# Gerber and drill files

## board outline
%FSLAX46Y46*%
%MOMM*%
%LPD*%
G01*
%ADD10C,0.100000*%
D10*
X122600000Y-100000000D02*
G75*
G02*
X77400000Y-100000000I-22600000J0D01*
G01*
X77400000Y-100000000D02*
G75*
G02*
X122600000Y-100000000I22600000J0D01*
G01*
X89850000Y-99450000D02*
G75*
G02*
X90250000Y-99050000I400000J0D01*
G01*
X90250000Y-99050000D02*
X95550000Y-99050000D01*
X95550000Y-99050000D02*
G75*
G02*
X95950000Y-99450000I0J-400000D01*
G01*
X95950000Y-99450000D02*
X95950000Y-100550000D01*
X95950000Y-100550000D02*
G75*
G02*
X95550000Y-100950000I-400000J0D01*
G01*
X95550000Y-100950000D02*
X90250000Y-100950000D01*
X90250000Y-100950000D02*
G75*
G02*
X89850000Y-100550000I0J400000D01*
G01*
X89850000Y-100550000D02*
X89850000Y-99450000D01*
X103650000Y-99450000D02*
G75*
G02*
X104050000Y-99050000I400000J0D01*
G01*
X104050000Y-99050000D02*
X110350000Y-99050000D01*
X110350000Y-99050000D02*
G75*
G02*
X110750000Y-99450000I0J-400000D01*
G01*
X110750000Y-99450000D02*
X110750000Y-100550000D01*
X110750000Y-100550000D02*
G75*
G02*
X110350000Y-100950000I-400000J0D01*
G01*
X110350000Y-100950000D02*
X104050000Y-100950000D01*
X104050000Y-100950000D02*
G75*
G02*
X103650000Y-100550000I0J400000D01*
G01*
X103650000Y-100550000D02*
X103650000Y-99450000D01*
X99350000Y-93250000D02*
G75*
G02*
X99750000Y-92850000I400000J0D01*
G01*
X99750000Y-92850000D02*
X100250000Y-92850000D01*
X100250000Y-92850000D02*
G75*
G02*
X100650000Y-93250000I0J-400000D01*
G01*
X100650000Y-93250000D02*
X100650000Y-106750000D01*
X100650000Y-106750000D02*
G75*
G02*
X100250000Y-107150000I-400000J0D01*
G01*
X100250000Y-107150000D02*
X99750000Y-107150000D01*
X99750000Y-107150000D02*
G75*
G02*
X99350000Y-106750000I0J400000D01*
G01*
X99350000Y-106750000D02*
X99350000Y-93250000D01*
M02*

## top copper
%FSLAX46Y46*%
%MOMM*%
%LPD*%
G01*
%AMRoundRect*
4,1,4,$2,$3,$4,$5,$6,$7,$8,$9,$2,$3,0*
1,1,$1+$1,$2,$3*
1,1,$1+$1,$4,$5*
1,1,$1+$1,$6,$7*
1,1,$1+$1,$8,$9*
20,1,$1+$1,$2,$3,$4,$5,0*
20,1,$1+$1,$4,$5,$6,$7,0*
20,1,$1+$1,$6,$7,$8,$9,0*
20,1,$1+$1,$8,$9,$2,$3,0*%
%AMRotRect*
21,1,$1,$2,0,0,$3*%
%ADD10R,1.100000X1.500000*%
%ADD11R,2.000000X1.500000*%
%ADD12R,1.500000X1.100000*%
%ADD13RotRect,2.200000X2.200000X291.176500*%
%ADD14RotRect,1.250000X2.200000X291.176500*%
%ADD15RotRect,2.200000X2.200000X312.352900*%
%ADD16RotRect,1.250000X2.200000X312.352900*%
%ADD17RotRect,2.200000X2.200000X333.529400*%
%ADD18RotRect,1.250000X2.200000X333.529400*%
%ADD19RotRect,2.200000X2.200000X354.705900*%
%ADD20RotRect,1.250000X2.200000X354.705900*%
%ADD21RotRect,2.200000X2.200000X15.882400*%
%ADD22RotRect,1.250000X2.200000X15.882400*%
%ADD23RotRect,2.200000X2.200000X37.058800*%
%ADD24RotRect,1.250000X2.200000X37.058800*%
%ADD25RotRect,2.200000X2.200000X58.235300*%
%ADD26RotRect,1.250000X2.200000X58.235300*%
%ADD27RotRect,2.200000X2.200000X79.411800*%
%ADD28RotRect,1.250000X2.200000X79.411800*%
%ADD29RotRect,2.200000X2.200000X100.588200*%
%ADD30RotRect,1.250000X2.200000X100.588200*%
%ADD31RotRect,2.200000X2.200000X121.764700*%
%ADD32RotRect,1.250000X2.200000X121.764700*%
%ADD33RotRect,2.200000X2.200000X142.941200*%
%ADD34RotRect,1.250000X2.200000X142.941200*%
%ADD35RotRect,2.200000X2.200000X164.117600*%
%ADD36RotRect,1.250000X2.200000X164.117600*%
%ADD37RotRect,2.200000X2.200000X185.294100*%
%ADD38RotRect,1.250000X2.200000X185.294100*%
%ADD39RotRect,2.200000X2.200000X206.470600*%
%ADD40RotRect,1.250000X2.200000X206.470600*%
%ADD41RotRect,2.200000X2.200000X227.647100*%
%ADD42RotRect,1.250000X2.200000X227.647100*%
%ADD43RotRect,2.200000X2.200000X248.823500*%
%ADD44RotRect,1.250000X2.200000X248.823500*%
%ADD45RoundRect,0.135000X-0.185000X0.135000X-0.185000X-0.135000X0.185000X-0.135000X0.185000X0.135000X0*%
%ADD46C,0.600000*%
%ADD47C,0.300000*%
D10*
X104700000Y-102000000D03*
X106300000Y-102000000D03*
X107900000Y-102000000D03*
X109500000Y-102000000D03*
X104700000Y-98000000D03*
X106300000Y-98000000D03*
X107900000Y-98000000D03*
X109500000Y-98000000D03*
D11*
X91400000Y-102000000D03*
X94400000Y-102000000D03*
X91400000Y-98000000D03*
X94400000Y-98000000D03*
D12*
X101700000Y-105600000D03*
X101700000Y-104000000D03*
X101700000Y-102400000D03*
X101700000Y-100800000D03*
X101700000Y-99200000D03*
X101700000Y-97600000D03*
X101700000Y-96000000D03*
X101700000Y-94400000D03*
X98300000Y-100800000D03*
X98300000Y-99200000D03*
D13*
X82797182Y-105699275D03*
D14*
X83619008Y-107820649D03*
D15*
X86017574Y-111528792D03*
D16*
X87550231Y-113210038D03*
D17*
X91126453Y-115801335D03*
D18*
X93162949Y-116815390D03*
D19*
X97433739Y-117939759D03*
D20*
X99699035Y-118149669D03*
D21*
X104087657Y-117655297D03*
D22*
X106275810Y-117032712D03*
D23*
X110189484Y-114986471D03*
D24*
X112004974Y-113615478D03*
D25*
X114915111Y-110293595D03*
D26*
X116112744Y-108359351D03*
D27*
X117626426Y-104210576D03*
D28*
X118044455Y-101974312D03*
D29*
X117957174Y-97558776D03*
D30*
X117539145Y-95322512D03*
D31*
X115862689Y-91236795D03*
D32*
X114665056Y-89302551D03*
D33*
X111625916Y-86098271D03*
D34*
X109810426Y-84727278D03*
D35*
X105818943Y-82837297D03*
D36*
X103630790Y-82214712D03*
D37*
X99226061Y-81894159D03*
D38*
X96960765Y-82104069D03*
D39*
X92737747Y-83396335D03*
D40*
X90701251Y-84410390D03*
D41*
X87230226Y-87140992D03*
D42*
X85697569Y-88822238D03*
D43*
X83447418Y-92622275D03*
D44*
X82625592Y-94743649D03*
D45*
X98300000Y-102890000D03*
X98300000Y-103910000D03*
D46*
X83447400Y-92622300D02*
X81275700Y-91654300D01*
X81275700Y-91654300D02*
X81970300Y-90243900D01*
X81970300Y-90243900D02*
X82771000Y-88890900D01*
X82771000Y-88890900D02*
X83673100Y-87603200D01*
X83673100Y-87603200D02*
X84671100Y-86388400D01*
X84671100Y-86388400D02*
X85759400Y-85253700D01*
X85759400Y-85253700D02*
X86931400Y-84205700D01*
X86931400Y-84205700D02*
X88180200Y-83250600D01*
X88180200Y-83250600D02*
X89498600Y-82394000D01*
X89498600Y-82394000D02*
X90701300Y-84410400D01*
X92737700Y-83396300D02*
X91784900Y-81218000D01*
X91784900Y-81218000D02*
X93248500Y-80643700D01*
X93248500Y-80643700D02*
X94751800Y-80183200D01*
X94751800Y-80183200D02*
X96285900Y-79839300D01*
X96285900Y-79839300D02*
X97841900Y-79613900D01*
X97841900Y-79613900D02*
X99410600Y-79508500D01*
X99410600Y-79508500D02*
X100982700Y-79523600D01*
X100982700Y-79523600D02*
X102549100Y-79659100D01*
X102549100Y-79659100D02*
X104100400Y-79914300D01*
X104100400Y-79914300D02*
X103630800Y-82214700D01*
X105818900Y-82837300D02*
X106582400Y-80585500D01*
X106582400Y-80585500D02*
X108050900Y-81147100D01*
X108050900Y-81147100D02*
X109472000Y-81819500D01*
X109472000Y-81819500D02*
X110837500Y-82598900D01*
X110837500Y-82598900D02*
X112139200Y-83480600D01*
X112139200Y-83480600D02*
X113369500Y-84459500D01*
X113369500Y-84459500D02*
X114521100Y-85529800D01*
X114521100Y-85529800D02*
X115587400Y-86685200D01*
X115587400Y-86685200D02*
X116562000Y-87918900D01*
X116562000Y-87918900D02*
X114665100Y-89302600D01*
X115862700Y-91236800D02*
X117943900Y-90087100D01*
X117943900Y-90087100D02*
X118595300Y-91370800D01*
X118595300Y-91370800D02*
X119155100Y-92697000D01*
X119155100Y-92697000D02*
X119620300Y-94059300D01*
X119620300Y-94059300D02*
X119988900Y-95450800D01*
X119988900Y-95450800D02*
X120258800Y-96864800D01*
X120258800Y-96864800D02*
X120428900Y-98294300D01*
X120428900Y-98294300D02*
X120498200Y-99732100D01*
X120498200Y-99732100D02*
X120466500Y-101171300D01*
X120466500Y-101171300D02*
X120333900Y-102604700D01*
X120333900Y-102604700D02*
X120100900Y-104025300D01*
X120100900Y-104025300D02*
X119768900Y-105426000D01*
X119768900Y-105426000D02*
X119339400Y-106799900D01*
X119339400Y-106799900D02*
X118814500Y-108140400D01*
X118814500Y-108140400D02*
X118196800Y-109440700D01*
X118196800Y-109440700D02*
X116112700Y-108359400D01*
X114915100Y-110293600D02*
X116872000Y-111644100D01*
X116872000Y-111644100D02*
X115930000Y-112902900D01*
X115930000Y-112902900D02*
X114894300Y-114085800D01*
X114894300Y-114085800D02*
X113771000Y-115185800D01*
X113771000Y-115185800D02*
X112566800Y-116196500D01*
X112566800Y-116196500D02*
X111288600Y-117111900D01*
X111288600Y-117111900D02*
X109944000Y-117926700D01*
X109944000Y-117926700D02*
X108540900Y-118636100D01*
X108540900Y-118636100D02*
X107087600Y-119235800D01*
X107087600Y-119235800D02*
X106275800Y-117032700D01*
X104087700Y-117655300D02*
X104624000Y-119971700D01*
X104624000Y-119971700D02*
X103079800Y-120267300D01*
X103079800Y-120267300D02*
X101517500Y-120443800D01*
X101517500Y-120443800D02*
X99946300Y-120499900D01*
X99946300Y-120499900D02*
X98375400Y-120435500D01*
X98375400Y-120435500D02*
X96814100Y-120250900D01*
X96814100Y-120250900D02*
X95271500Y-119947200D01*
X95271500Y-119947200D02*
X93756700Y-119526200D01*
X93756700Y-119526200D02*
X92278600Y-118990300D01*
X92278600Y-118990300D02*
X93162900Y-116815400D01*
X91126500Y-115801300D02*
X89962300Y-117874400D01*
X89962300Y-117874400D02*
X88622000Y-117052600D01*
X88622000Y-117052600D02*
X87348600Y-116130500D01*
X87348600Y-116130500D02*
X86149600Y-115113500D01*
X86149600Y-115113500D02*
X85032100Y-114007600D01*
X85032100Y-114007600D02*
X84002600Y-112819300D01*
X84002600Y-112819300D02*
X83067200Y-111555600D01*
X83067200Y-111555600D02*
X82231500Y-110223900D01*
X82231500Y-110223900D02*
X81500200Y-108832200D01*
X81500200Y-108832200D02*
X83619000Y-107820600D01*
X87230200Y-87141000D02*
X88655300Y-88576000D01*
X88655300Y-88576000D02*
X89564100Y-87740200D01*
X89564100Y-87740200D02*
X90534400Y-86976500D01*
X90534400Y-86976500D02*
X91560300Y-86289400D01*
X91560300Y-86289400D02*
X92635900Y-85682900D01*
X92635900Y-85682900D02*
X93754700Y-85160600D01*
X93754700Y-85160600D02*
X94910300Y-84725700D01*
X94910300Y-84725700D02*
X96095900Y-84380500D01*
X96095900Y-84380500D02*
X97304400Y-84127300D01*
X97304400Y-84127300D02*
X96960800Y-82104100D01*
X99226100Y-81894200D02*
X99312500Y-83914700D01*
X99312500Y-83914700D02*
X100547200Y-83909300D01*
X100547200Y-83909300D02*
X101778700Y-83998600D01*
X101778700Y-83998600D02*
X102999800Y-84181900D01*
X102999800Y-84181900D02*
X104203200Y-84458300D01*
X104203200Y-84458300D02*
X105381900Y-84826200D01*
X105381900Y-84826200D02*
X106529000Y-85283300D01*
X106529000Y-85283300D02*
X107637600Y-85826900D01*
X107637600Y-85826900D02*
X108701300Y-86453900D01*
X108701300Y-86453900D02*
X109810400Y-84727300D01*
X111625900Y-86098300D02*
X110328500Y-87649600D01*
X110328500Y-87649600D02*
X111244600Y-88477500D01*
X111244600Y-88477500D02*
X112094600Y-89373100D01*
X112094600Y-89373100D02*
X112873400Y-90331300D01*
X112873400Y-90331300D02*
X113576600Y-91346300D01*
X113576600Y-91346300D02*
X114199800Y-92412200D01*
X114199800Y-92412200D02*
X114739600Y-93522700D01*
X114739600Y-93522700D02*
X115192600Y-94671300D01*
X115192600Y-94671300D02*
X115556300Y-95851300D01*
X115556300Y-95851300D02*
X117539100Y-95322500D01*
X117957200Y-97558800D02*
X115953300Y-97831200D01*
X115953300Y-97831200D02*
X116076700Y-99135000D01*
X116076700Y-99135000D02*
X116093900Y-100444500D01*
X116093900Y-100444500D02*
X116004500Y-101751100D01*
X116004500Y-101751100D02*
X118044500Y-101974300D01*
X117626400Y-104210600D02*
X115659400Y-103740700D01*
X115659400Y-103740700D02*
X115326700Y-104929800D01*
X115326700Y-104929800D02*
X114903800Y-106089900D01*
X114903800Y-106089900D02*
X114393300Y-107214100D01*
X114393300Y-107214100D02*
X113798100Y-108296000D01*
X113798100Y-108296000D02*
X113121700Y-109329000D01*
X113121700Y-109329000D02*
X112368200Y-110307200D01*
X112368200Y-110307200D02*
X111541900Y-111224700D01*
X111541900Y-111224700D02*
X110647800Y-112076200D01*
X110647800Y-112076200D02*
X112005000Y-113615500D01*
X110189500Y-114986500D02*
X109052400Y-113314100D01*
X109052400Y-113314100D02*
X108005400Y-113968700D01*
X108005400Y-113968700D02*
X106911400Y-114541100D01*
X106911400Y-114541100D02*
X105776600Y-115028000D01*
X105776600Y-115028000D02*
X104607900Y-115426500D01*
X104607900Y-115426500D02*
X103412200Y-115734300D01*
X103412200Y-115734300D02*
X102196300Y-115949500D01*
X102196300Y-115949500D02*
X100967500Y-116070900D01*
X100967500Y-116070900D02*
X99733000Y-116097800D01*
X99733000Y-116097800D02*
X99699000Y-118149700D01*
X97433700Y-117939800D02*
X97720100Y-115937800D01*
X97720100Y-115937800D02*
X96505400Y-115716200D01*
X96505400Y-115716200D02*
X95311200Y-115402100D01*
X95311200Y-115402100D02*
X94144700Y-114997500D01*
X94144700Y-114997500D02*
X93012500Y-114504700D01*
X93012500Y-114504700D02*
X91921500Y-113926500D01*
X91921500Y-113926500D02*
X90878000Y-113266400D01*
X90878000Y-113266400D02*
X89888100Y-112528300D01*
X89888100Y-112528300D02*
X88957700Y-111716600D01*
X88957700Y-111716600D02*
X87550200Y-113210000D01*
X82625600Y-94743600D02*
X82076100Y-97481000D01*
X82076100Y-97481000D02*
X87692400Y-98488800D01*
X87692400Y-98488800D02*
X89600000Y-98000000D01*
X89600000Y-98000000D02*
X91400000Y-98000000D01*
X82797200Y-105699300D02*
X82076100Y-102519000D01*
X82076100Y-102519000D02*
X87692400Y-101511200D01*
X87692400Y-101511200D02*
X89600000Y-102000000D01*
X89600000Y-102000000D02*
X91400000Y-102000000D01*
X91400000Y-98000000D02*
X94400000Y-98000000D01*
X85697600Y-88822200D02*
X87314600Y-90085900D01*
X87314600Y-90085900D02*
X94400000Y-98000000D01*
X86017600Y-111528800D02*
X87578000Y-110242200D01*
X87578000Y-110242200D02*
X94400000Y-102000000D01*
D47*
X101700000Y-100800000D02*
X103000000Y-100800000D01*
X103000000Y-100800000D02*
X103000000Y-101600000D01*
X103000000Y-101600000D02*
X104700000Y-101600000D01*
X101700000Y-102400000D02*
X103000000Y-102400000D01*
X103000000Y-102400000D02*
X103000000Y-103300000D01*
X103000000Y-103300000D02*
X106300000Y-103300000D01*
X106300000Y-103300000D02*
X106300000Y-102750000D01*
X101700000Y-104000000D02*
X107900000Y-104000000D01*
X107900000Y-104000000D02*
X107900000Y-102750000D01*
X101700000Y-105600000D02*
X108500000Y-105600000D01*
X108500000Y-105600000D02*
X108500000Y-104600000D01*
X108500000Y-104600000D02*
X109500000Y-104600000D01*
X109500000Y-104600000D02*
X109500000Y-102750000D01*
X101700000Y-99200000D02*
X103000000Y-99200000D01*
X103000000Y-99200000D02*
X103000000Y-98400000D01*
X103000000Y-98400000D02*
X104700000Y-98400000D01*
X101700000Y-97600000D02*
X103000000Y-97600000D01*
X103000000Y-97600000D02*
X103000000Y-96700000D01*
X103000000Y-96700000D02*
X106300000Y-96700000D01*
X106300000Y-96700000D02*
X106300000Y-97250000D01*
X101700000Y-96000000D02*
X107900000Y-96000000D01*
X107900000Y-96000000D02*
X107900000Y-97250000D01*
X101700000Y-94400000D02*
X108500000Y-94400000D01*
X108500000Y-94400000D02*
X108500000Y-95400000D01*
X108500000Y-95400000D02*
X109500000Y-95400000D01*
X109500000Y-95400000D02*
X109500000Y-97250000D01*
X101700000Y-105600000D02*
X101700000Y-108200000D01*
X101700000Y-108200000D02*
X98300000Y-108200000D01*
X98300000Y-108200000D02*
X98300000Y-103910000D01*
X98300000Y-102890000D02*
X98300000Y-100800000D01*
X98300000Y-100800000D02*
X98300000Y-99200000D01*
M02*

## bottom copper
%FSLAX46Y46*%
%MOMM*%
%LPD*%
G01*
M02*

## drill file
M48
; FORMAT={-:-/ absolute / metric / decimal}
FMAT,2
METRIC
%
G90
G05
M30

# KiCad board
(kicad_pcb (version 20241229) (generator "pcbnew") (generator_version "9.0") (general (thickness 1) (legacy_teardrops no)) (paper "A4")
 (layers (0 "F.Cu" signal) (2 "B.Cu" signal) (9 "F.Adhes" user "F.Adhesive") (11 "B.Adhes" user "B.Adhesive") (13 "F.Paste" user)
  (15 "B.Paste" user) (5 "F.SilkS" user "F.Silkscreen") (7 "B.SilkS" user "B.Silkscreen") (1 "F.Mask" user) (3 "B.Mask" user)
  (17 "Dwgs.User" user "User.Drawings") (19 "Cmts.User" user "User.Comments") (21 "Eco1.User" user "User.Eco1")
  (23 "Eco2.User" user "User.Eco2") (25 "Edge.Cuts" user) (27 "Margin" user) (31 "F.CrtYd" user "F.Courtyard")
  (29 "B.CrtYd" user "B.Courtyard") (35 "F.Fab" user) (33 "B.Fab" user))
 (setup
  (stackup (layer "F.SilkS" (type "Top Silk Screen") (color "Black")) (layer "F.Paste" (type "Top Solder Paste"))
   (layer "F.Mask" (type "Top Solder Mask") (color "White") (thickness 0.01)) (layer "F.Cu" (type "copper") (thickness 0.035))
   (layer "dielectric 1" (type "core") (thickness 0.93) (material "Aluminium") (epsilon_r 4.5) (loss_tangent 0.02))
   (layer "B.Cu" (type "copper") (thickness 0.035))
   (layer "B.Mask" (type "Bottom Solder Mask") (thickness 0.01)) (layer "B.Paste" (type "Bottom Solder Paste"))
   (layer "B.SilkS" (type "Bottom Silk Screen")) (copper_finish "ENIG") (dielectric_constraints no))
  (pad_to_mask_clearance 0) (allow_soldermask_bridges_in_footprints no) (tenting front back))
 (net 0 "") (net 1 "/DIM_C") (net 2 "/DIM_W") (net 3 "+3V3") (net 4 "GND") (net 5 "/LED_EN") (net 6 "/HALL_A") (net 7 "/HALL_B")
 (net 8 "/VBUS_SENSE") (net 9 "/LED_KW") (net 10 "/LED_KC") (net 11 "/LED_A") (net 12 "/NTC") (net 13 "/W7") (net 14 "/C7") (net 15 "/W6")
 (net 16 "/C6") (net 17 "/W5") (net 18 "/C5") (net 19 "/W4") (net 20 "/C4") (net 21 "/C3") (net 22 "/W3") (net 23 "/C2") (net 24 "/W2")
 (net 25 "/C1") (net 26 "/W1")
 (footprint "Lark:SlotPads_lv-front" (layer "F.Cu") (at 100 100)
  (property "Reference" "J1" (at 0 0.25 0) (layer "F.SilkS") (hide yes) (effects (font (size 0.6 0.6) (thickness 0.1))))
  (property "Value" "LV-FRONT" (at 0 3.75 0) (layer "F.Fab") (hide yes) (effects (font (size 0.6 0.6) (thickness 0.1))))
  (pad "1" smd rect (at 4.7 2) (size 1.1 1.5) (layers "F.Cu" "F.Mask") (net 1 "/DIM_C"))
  (pad "2" smd rect (at 6.3 2) (size 1.1 1.5) (layers "F.Cu" "F.Mask") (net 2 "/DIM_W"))
  (pad "3" smd rect (at 7.9 2) (size 1.1 1.5) (layers "F.Cu" "F.Mask") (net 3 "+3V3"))
  (pad "4" smd rect (at 9.5 2) (size 1.1 1.5) (layers "F.Cu" "F.Mask") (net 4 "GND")))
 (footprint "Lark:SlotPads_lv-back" (layer "F.Cu") (at 100 100)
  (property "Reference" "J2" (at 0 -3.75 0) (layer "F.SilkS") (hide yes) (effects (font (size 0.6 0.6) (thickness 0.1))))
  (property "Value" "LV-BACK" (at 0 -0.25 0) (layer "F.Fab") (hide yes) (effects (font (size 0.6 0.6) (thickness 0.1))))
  (pad "1" smd rect (at 4.7 -2) (size 1.1 1.5) (layers "F.Cu" "F.Mask") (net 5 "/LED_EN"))
  (pad "2" smd rect (at 6.3 -2) (size 1.1 1.5) (layers "F.Cu" "F.Mask") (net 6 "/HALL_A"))
  (pad "3" smd rect (at 7.9 -2) (size 1.1 1.5) (layers "F.Cu" "F.Mask") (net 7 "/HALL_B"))
  (pad "4" smd rect (at 9.5 -2) (size 1.1 1.5) (layers "F.Cu" "F.Mask") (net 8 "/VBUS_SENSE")))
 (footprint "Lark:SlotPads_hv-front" (layer "F.Cu") (at 100 100)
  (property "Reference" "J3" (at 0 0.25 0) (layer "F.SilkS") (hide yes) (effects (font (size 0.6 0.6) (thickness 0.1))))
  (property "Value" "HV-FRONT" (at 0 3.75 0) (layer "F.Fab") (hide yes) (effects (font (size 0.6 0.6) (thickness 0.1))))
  (pad "1" smd rect (at -8.6 2) (size 2 1.5) (layers "F.Cu" "F.Mask") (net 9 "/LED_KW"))
  (pad "2" smd rect (at -5.6 2) (size 2 1.5) (layers "F.Cu" "F.Mask") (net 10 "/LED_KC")))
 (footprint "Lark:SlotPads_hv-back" (layer "F.Cu") (at 100 100)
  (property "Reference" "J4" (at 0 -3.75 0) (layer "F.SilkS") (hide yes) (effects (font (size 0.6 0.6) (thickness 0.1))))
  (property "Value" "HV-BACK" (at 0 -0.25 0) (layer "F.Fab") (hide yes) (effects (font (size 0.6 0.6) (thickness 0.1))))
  (pad "1" smd rect (at -8.6 -2) (size 2 1.5) (layers "F.Cu" "F.Mask") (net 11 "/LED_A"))
  (pad "2" smd rect (at -5.6 -2) (size 2 1.5) (layers "F.Cu" "F.Mask") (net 11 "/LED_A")))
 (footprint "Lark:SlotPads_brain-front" (layer "F.Cu") (at 100 100)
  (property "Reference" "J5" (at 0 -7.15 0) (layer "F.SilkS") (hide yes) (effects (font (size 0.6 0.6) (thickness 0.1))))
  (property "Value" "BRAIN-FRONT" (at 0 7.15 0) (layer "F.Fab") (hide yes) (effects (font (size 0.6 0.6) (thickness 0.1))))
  (pad "1" smd rect (at 1.7 5.6) (size 1.5 1.1) (layers "F.Cu" "F.Mask") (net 4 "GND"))
  (pad "2" smd rect (at 1.7 4) (size 1.5 1.1) (layers "F.Cu" "F.Mask") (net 3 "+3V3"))
  (pad "3" smd rect (at 1.7 2.4) (size 1.5 1.1) (layers "F.Cu" "F.Mask") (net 2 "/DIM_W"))
  (pad "4" smd rect (at 1.7 0.8) (size 1.5 1.1) (layers "F.Cu" "F.Mask") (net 1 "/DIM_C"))
  (pad "5" smd rect (at 1.7 -0.8) (size 1.5 1.1) (layers "F.Cu" "F.Mask") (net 5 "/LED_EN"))
  (pad "6" smd rect (at 1.7 -2.4) (size 1.5 1.1) (layers "F.Cu" "F.Mask") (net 6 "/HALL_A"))
  (pad "7" smd rect (at 1.7 -4) (size 1.5 1.1) (layers "F.Cu" "F.Mask") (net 7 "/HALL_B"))
  (pad "8" smd rect (at 1.7 -5.6) (size 1.5 1.1) (layers "F.Cu" "F.Mask") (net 8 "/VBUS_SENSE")))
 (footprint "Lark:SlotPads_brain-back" (layer "F.Cu") (at 100 100)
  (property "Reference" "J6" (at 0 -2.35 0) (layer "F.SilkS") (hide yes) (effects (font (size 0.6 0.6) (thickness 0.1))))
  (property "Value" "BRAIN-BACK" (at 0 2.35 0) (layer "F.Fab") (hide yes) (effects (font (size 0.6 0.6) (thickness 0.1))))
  (pad "1" smd rect (at -1.7 0.8) (size 1.5 1.1) (layers "F.Cu" "F.Mask") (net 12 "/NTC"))
  (pad "2" smd rect (at -1.7 -0.8) (size 1.5 1.1) (layers "F.Cu" "F.Mask") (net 12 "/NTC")))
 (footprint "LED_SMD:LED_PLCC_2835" (layer "F.Cu") (at 83.1223 106.5385 291.1765)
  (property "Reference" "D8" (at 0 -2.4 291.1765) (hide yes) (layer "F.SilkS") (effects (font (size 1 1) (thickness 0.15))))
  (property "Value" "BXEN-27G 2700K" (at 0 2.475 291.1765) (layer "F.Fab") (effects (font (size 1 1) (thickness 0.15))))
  (pad "1" smd rect (at -0.9 0 291.1765) (size 2.2 2.2) (layers "F.Cu" "F.Mask" "F.Paste") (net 9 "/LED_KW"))
  (pad "2" smd rect (at 1.375 0 291.1765) (size 1.25 2.2) (layers "F.Cu" "F.Mask" "F.Paste") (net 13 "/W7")))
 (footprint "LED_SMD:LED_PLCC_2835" (layer "F.Cu") (at 86.6239 112.1939 312.3529)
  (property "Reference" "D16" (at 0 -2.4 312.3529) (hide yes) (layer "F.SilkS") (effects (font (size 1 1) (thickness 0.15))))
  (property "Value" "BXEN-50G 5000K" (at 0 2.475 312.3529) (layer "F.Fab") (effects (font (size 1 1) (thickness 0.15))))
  (pad "1" smd rect (at -0.9 0 312.3529) (size 2.2 2.2) (layers "F.Cu" "F.Mask" "F.Paste") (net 10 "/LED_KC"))
  (pad "2" smd rect (at 1.375 0 312.3529) (size 1.25 2.2) (layers "F.Cu" "F.Mask" "F.Paste") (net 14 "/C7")))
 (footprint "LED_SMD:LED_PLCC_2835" (layer "F.Cu") (at 91.9321 116.2025 333.5294)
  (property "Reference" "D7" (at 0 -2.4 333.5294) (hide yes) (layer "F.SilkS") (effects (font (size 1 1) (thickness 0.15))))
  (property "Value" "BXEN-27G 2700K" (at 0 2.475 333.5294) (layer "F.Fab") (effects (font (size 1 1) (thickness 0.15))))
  (pad "1" smd rect (at -0.9 0 333.5294) (size 2.2 2.2) (layers "F.Cu" "F.Mask" "F.Paste") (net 13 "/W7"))
  (pad "2" smd rect (at 1.375 0 333.5294) (size 1.25 2.2) (layers "F.Cu" "F.Mask" "F.Paste") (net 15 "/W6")))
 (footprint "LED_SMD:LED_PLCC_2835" (layer "F.Cu") (at 98.3299 118.0228 354.7059)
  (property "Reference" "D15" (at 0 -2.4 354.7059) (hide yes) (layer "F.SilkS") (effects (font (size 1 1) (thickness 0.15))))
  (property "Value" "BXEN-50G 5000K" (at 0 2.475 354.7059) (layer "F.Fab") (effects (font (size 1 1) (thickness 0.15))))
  (pad "1" smd rect (at -0.9 0 354.7059) (size 2.2 2.2) (layers "F.Cu" "F.Mask" "F.Paste") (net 14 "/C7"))
  (pad "2" smd rect (at 1.375 0 354.7059) (size 1.25 2.2) (layers "F.Cu" "F.Mask" "F.Paste") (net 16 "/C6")))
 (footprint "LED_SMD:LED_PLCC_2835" (layer "F.Cu") (at 104.9533 117.409 15.8824)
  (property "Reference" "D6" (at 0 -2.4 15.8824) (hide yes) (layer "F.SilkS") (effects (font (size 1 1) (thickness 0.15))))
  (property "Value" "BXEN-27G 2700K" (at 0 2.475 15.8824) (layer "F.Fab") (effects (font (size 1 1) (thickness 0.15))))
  (pad "1" smd rect (at -0.9 0 15.8824) (size 2.2 2.2) (layers "F.Cu" "F.Mask" "F.Paste") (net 15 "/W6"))
  (pad "2" smd rect (at 1.375 0 15.8824) (size 1.25 2.2) (layers "F.Cu" "F.Mask" "F.Paste") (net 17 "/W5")))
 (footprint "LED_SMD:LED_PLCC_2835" (layer "F.Cu") (at 110.9077 114.4441 37.0588)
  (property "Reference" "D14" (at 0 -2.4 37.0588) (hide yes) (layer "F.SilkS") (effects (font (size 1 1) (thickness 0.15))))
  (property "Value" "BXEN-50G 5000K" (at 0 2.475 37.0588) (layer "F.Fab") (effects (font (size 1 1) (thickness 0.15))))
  (pad "1" smd rect (at -0.9 0 37.0588) (size 2.2 2.2) (layers "F.Cu" "F.Mask" "F.Paste") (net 16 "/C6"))
  (pad "2" smd rect (at 1.375 0 37.0588) (size 1.25 2.2) (layers "F.Cu" "F.Mask" "F.Paste") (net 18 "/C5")))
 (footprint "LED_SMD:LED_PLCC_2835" (layer "F.Cu") (at 115.3889 109.5284 58.2353)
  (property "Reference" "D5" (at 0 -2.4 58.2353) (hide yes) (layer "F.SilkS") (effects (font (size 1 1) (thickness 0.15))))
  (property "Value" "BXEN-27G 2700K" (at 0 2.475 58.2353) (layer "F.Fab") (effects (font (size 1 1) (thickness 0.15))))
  (pad "1" smd rect (at -0.9 0 58.2353) (size 2.2 2.2) (layers "F.Cu" "F.Mask" "F.Paste") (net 17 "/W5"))
  (pad "2" smd rect (at 1.375 0 58.2353) (size 1.25 2.2) (layers "F.Cu" "F.Mask" "F.Paste") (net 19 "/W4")))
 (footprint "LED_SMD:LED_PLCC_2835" (layer "F.Cu") (at 117.7918 103.3259 79.4118)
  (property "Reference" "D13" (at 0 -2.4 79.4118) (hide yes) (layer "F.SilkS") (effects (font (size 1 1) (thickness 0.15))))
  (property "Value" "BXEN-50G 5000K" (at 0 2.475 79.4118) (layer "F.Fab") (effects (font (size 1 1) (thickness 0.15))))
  (pad "1" smd rect (at -0.9 0 79.4118) (size 2.2 2.2) (layers "F.Cu" "F.Mask" "F.Paste") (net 18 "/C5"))
  (pad "2" smd rect (at 1.375 0 79.4118) (size 1.25 2.2) (layers "F.Cu" "F.Mask" "F.Paste") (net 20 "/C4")))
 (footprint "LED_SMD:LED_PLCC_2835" (layer "F.Cu") (at 117.7918 96.6741 100.5882)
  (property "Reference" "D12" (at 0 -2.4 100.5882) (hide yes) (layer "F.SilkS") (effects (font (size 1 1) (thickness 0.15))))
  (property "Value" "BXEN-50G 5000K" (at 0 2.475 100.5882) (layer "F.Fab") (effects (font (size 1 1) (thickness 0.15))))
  (pad "1" smd rect (at -0.9 0 100.5882) (size 2.2 2.2) (layers "F.Cu" "F.Mask" "F.Paste") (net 20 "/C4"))
  (pad "2" smd rect (at 1.375 0 100.5882) (size 1.25 2.2) (layers "F.Cu" "F.Mask" "F.Paste") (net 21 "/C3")))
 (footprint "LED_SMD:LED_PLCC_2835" (layer "F.Cu") (at 115.3889 90.4716 121.7647)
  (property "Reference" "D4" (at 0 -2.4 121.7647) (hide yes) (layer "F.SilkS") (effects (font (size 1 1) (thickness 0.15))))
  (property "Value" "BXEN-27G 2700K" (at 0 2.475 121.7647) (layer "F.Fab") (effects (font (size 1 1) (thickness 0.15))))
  (pad "1" smd rect (at -0.9 0 121.7647) (size 2.2 2.2) (layers "F.Cu" "F.Mask" "F.Paste") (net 19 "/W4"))
  (pad "2" smd rect (at 1.375 0 121.7647) (size 1.25 2.2) (layers "F.Cu" "F.Mask" "F.Paste") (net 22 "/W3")))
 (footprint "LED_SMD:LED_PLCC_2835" (layer "F.Cu") (at 110.9077 85.5559 142.9412)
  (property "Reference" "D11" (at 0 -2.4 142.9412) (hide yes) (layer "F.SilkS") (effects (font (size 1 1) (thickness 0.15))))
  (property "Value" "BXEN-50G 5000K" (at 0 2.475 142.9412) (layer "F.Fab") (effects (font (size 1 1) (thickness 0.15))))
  (pad "1" smd rect (at -0.9 0 142.9412) (size 2.2 2.2) (layers "F.Cu" "F.Mask" "F.Paste") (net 21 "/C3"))
  (pad "2" smd rect (at 1.375 0 142.9412) (size 1.25 2.2) (layers "F.Cu" "F.Mask" "F.Paste") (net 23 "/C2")))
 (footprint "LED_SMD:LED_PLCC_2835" (layer "F.Cu") (at 104.9533 82.591 164.1176)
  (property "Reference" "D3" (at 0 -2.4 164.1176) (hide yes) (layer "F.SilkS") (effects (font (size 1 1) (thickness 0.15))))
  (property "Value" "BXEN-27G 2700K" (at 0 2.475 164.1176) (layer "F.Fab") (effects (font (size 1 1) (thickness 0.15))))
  (pad "1" smd rect (at -0.9 0 164.1176) (size 2.2 2.2) (layers "F.Cu" "F.Mask" "F.Paste") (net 22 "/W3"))
  (pad "2" smd rect (at 1.375 0 164.1176) (size 1.25 2.2) (layers "F.Cu" "F.Mask" "F.Paste") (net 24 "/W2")))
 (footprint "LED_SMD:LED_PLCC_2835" (layer "F.Cu") (at 98.3299 81.9772 185.2941)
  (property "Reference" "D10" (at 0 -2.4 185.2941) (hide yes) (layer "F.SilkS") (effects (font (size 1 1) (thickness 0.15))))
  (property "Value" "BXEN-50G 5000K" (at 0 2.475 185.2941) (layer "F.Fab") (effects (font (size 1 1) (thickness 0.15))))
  (pad "1" smd rect (at -0.9 0 185.2941) (size 2.2 2.2) (layers "F.Cu" "F.Mask" "F.Paste") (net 23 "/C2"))
  (pad "2" smd rect (at 1.375 0 185.2941) (size 1.25 2.2) (layers "F.Cu" "F.Mask" "F.Paste") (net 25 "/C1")))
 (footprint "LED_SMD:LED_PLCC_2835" (layer "F.Cu") (at 91.9321 83.7975 206.4706)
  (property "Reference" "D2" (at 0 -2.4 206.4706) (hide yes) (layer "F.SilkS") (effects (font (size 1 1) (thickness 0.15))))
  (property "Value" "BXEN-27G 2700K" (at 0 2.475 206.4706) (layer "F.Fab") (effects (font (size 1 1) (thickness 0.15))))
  (pad "1" smd rect (at -0.9 0 206.4706) (size 2.2 2.2) (layers "F.Cu" "F.Mask" "F.Paste") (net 24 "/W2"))
  (pad "2" smd rect (at 1.375 0 206.4706) (size 1.25 2.2) (layers "F.Cu" "F.Mask" "F.Paste") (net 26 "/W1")))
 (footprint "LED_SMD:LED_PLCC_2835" (layer "F.Cu") (at 86.6239 87.8061 227.6471)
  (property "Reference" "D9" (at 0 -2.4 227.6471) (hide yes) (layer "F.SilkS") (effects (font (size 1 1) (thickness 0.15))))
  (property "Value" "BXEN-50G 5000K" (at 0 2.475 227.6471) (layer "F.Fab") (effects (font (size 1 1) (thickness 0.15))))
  (pad "1" smd rect (at -0.9 0 227.6471) (size 2.2 2.2) (layers "F.Cu" "F.Mask" "F.Paste") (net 25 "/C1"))
  (pad "2" smd rect (at 1.375 0 227.6471) (size 1.25 2.2) (layers "F.Cu" "F.Mask" "F.Paste") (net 11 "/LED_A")))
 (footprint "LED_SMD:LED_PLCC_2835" (layer "F.Cu") (at 83.1223 93.4615 248.8235)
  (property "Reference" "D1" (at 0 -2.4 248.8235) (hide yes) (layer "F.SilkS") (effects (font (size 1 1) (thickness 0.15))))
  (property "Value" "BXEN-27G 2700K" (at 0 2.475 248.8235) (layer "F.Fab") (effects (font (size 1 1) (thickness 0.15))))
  (pad "1" smd rect (at -0.9 0 248.8235) (size 2.2 2.2) (layers "F.Cu" "F.Mask" "F.Paste") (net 26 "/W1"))
  (pad "2" smd rect (at 1.375 0 248.8235) (size 1.25 2.2) (layers "F.Cu" "F.Mask" "F.Paste") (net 11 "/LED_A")))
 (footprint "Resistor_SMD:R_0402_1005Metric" (layer "F.Cu") (at 98.3 103.4 270)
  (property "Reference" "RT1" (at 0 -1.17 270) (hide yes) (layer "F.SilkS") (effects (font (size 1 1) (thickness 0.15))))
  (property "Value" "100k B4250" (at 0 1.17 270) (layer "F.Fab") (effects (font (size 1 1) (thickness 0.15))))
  (pad "1" smd roundrect (at -0.51 0 270) (size 0.54 0.64) (layers "F.Cu" "F.Mask" "F.Paste") (roundrect_rratio 0.25) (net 12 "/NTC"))
  (pad "2" smd roundrect (at 0.51 0 270) (size 0.54 0.64) (layers "F.Cu" "F.Mask" "F.Paste") (roundrect_rratio 0.25) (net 4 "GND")))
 (gr_circle (center 100 100) (end 122.6 100) (stroke (width 0.1) (type default)) (fill no) (layer "Edge.Cuts"))
 (gr_arc (start 89.85 99.45) (mid 89.967157 99.167157) (end 90.25 99.05) (stroke (width 0.1) (type default)) (layer "Edge.Cuts"))
 (gr_line (start 90.25 99.05) (end 95.55 99.05) (stroke (width 0.1) (type default)) (layer "Edge.Cuts"))
 (gr_arc (start 95.55 99.05) (mid 95.832843 99.167157) (end 95.95 99.45) (stroke (width 0.1) (type default)) (layer "Edge.Cuts"))
 (gr_line (start 95.95 99.45) (end 95.95 100.55) (stroke (width 0.1) (type default)) (layer "Edge.Cuts"))
 (gr_arc (start 95.95 100.55) (mid 95.832843 100.832843) (end 95.55 100.95) (stroke (width 0.1) (type default)) (layer "Edge.Cuts"))
 (gr_line (start 95.55 100.95) (end 90.25 100.95) (stroke (width 0.1) (type default)) (layer "Edge.Cuts"))
 (gr_arc (start 90.25 100.95) (mid 89.967157 100.832843) (end 89.85 100.55) (stroke (width 0.1) (type default)) (layer "Edge.Cuts"))
 (gr_line (start 89.85 100.55) (end 89.85 99.45) (stroke (width 0.1) (type default)) (layer "Edge.Cuts"))
 (gr_arc (start 103.65 99.45) (mid 103.767157 99.167157) (end 104.05 99.05) (stroke (width 0.1) (type default)) (layer "Edge.Cuts"))
 (gr_line (start 104.05 99.05) (end 110.35 99.05) (stroke (width 0.1) (type default)) (layer "Edge.Cuts"))
 (gr_arc (start 110.35 99.05) (mid 110.632843 99.167157) (end 110.75 99.45) (stroke (width 0.1) (type default)) (layer "Edge.Cuts"))
 (gr_line (start 110.75 99.45) (end 110.75 100.55) (stroke (width 0.1) (type default)) (layer "Edge.Cuts"))
 (gr_arc (start 110.75 100.55) (mid 110.632843 100.832843) (end 110.35 100.95) (stroke (width 0.1) (type default)) (layer "Edge.Cuts"))
 (gr_line (start 110.35 100.95) (end 104.05 100.95) (stroke (width 0.1) (type default)) (layer "Edge.Cuts"))
 (gr_arc (start 104.05 100.95) (mid 103.767157 100.832843) (end 103.65 100.55) (stroke (width 0.1) (type default)) (layer "Edge.Cuts"))
 (gr_line (start 103.65 100.55) (end 103.65 99.45) (stroke (width 0.1) (type default)) (layer "Edge.Cuts"))
 (gr_arc (start 99.35 93.25) (mid 99.467157 92.967157) (end 99.75 92.85) (stroke (width 0.1) (type default)) (layer "Edge.Cuts"))
 (gr_line (start 99.75 92.85) (end 100.25 92.85) (stroke (width 0.1) (type default)) (layer "Edge.Cuts"))
 (gr_arc (start 100.25 92.85) (mid 100.532843 92.967157) (end 100.65 93.25) (stroke (width 0.1) (type default)) (layer "Edge.Cuts"))
 (gr_line (start 100.65 93.25) (end 100.65 106.75) (stroke (width 0.1) (type default)) (layer "Edge.Cuts"))
 (gr_arc (start 100.65 106.75) (mid 100.532843 107.032843) (end 100.25 107.15) (stroke (width 0.1) (type default)) (layer "Edge.Cuts"))
 (gr_line (start 100.25 107.15) (end 99.75 107.15) (stroke (width 0.1) (type default)) (layer "Edge.Cuts"))
 (gr_arc (start 99.75 107.15) (mid 99.467157 107.032843) (end 99.35 106.75) (stroke (width 0.1) (type default)) (layer "Edge.Cuts"))
 (gr_line (start 99.35 106.75) (end 99.35 93.25) (stroke (width 0.1) (type default)) (layer "Edge.Cuts"))
 (segment (start 83.4474 92.6223) (end 81.2757 91.6543) (width 0.6) (layer "F.Cu") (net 26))
 (segment (start 81.2757 91.6543) (end 81.9703 90.2439) (width 0.6) (layer "F.Cu") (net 26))
 (segment (start 81.9703 90.2439) (end 82.771 88.8909) (width 0.6) (layer "F.Cu") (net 26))
 (segment (start 82.771 88.8909) (end 83.6731 87.6032) (width 0.6) (layer "F.Cu") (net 26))
 (segment (start 83.6731 87.6032) (end 84.6711 86.3884) (width 0.6) (layer "F.Cu") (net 26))
 (segment (start 84.6711 86.3884) (end 85.7594 85.2537) (width 0.6) (layer "F.Cu") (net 26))
 (segment (start 85.7594 85.2537) (end 86.9314 84.2057) (width 0.6) (layer "F.Cu") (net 26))
 (segment (start 86.9314 84.2057) (end 88.1802 83.2506) (width 0.6) (layer "F.Cu") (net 26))
 (segment (start 88.1802 83.2506) (end 89.4986 82.394) (width 0.6) (layer "F.Cu") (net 26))
 (segment (start 89.4986 82.394) (end 90.7013 84.4104) (width 0.6) (layer "F.Cu") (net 26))
 (segment (start 92.7377 83.3963) (end 91.7849 81.218) (width 0.6) (layer "F.Cu") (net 24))
 (segment (start 91.7849 81.218) (end 93.2485 80.6437) (width 0.6) (layer "F.Cu") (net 24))
 (segment (start 93.2485 80.6437) (end 94.7518 80.1832) (width 0.6) (layer "F.Cu") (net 24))
 (segment (start 94.7518 80.1832) (end 96.2859 79.8393) (width 0.6) (layer "F.Cu") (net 24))
 (segment (start 96.2859 79.8393) (end 97.8419 79.6139) (width 0.6) (layer "F.Cu") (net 24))
 (segment (start 97.8419 79.6139) (end 99.4106 79.5085) (width 0.6) (layer "F.Cu") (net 24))
 (segment (start 99.4106 79.5085) (end 100.9827 79.5236) (width 0.6) (layer "F.Cu") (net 24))
 (segment (start 100.9827 79.5236) (end 102.5491 79.6591) (width 0.6) (layer "F.Cu") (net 24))
 (segment (start 102.5491 79.6591) (end 104.1004 79.9143) (width 0.6) (layer "F.Cu") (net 24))
 (segment (start 104.1004 79.9143) (end 103.6308 82.2147) (width 0.6) (layer "F.Cu") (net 24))
 (segment (start 105.8189 82.8373) (end 106.5824 80.5855) (width 0.6) (layer "F.Cu") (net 22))
 (segment (start 106.5824 80.5855) (end 108.0509 81.1471) (width 0.6) (layer "F.Cu") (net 22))
 (segment (start 108.0509 81.1471) (end 109.472 81.8195) (width 0.6) (layer "F.Cu") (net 22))
 (segment (start 109.472 81.8195) (end 110.8375 82.5989) (width 0.6) (layer "F.Cu") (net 22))
 (segment (start 110.8375 82.5989) (end 112.1392 83.4806) (width 0.6) (layer "F.Cu") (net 22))
 (segment (start 112.1392 83.4806) (end 113.3695 84.4595) (width 0.6) (layer "F.Cu") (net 22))
 (segment (start 113.3695 84.4595) (end 114.5211 85.5298) (width 0.6) (layer "F.Cu") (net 22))
 (segment (start 114.5211 85.5298) (end 115.5874 86.6852) (width 0.6) (layer "F.Cu") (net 22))
 (segment (start 115.5874 86.6852) (end 116.562 87.9189) (width 0.6) (layer "F.Cu") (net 22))
 (segment (start 116.562 87.9189) (end 114.6651 89.3026) (width 0.6) (layer "F.Cu") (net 22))
 (segment (start 115.8627 91.2368) (end 117.9439 90.0871) (width 0.6) (layer "F.Cu") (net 19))
 (segment (start 117.9439 90.0871) (end 118.5953 91.3708) (width 0.6) (layer "F.Cu") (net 19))
 (segment (start 118.5953 91.3708) (end 119.1551 92.697) (width 0.6) (layer "F.Cu") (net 19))
 (segment (start 119.1551 92.697) (end 119.6203 94.0593) (width 0.6) (layer "F.Cu") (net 19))
 (segment (start 119.6203 94.0593) (end 119.9889 95.4508) (width 0.6) (layer "F.Cu") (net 19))
 (segment (start 119.9889 95.4508) (end 120.2588 96.8648) (width 0.6) (layer "F.Cu") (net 19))
 (segment (start 120.2588 96.8648) (end 120.4289 98.2943) (width 0.6) (layer "F.Cu") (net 19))
 (segment (start 120.4289 98.2943) (end 120.4982 99.7321) (width 0.6) (layer "F.Cu") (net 19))
 (segment (start 120.4982 99.7321) (end 120.4665 101.1713) (width 0.6) (layer "F.Cu") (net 19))
 (segment (start 120.4665 101.1713) (end 120.3339 102.6047) (width 0.6) (layer "F.Cu") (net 19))
 (segment (start 120.3339 102.6047) (end 120.1009 104.0253) (width 0.6) (layer "F.Cu") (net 19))
 (segment (start 120.1009 104.0253) (end 119.7689 105.426) (width 0.6) (layer "F.Cu") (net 19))
 (segment (start 119.7689 105.426) (end 119.3394 106.7999) (width 0.6) (layer "F.Cu") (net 19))
 (segment (start 119.3394 106.7999) (end 118.8145 108.1404) (width 0.6) (layer "F.Cu") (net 19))
 (segment (start 118.8145 108.1404) (end 118.1968 109.4407) (width 0.6) (layer "F.Cu") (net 19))
 (segment (start 118.1968 109.4407) (end 116.1127 108.3594) (width 0.6) (layer "F.Cu") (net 19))
 (segment (start 114.9151 110.2936) (end 116.872 111.6441) (width 0.6) (layer "F.Cu") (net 17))
 (segment (start 116.872 111.6441) (end 115.93 112.9029) (width 0.6) (layer "F.Cu") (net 17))
 (segment (start 115.93 112.9029) (end 114.8943 114.0858) (width 0.6) (layer "F.Cu") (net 17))
 (segment (start 114.8943 114.0858) (end 113.771 115.1858) (width 0.6) (layer "F.Cu") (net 17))
 (segment (start 113.771 115.1858) (end 112.5668 116.1965) (width 0.6) (layer "F.Cu") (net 17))
 (segment (start 112.5668 116.1965) (end 111.2886 117.1119) (width 0.6) (layer "F.Cu") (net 17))
 (segment (start 111.2886 117.1119) (end 109.944 117.9267) (width 0.6) (layer "F.Cu") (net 17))
 (segment (start 109.944 117.9267) (end 108.5409 118.6361) (width 0.6) (layer "F.Cu") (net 17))
 (segment (start 108.5409 118.6361) (end 107.0876 119.2358) (width 0.6) (layer "F.Cu") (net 17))
 (segment (start 107.0876 119.2358) (end 106.2758 117.0327) (width 0.6) (layer "F.Cu") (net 17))
 (segment (start 104.0877 117.6553) (end 104.624 119.9717) (width 0.6) (layer "F.Cu") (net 15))
 (segment (start 104.624 119.9717) (end 103.0798 120.2673) (width 0.6) (layer "F.Cu") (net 15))
 (segment (start 103.0798 120.2673) (end 101.5175 120.4438) (width 0.6) (layer "F.Cu") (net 15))
 (segment (start 101.5175 120.4438) (end 99.9463 120.4999) (width 0.6) (layer "F.Cu") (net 15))
 (segment (start 99.9463 120.4999) (end 98.3754 120.4355) (width 0.6) (layer "F.Cu") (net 15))
 (segment (start 98.3754 120.4355) (end 96.8141 120.2509) (width 0.6) (layer "F.Cu") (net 15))
 (segment (start 96.8141 120.2509) (end 95.2715 119.9472) (width 0.6) (layer "F.Cu") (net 15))
 (segment (start 95.2715 119.9472) (end 93.7567 119.5262) (width 0.6) (layer "F.Cu") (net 15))
 (segment (start 93.7567 119.5262) (end 92.2786 118.9903) (width 0.6) (layer "F.Cu") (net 15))
 (segment (start 92.2786 118.9903) (end 93.1629 116.8154) (width 0.6) (layer "F.Cu") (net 15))
 (segment (start 91.1265 115.8013) (end 89.9623 117.8744) (width 0.6) (layer "F.Cu") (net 13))
 (segment (start 89.9623 117.8744) (end 88.622 117.0526) (width 0.6) (layer "F.Cu") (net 13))
 (segment (start 88.622 117.0526) (end 87.3486 116.1305) (width 0.6) (layer "F.Cu") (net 13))
 (segment (start 87.3486 116.1305) (end 86.1496 115.1135) (width 0.6) (layer "F.Cu") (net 13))
 (segment (start 86.1496 115.1135) (end 85.0321 114.0076) (width 0.6) (layer "F.Cu") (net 13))
 (segment (start 85.0321 114.0076) (end 84.0026 112.8193) (width 0.6) (layer "F.Cu") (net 13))
 (segment (start 84.0026 112.8193) (end 83.0672 111.5556) (width 0.6) (layer "F.Cu") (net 13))
 (segment (start 83.0672 111.5556) (end 82.2315 110.2239) (width 0.6) (layer "F.Cu") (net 13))
 (segment (start 82.2315 110.2239) (end 81.5002 108.8322) (width 0.6) (layer "F.Cu") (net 13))
 (segment (start 81.5002 108.8322) (end 83.619 107.8206) (width 0.6) (layer "F.Cu") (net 13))
 (segment (start 87.2302 87.141) (end 88.6553 88.576) (width 0.6) (layer "F.Cu") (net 25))
 (segment (start 88.6553 88.576) (end 89.5641 87.7402) (width 0.6) (layer "F.Cu") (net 25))
 (segment (start 89.5641 87.7402) (end 90.5344 86.9765) (width 0.6) (layer "F.Cu") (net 25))
 (segment (start 90.5344 86.9765) (end 91.5603 86.2894) (width 0.6) (layer "F.Cu") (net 25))
 (segment (start 91.5603 86.2894) (end 92.6359 85.6829) (width 0.6) (layer "F.Cu") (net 25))
 (segment (start 92.6359 85.6829) (end 93.7547 85.1606) (width 0.6) (layer "F.Cu") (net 25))
 (segment (start 93.7547 85.1606) (end 94.9103 84.7257) (width 0.6) (layer "F.Cu") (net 25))
 (segment (start 94.9103 84.7257) (end 96.0959 84.3805) (width 0.6) (layer "F.Cu") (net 25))
 (segment (start 96.0959 84.3805) (end 97.3044 84.1273) (width 0.6) (layer "F.Cu") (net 25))
 (segment (start 97.3044 84.1273) (end 96.9608 82.1041) (width 0.6) (layer "F.Cu") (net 25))
 (segment (start 99.2261 81.8942) (end 99.3125 83.9147) (width 0.6) (layer "F.Cu") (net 23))
 (segment (start 99.3125 83.9147) (end 100.5472 83.9093) (width 0.6) (layer "F.Cu") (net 23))
 (segment (start 100.5472 83.9093) (end 101.7787 83.9986) (width 0.6) (layer "F.Cu") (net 23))
 (segment (start 101.7787 83.9986) (end 102.9998 84.1819) (width 0.6) (layer "F.Cu") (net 23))
 (segment (start 102.9998 84.1819) (end 104.2032 84.4583) (width 0.6) (layer "F.Cu") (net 23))
 (segment (start 104.2032 84.4583) (end 105.3819 84.8262) (width 0.6) (layer "F.Cu") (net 23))
 (segment (start 105.3819 84.8262) (end 106.529 85.2833) (width 0.6) (layer "F.Cu") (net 23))
 (segment (start 106.529 85.2833) (end 107.6376 85.8269) (width 0.6) (layer "F.Cu") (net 23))
 (segment (start 107.6376 85.8269) (end 108.7013 86.4539) (width 0.6) (layer "F.Cu") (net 23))
 (segment (start 108.7013 86.4539) (end 109.8104 84.7273) (width 0.6) (layer "F.Cu") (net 23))
 (segment (start 111.6259 86.0983) (end 110.3285 87.6496) (width 0.6) (layer "F.Cu") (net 21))
 (segment (start 110.3285 87.6496) (end 111.2446 88.4775) (width 0.6) (layer "F.Cu") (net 21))
 (segment (start 111.2446 88.4775) (end 112.0946 89.3731) (width 0.6) (layer "F.Cu") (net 21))
 (segment (start 112.0946 89.3731) (end 112.8734 90.3313) (width 0.6) (layer "F.Cu") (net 21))
 (segment (start 112.8734 90.3313) (end 113.5766 91.3463) (width 0.6) (layer "F.Cu") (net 21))
 (segment (start 113.5766 91.3463) (end 114.1998 92.4122) (width 0.6) (layer "F.Cu") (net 21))
 (segment (start 114.1998 92.4122) (end 114.7396 93.5227) (width 0.6) (layer "F.Cu") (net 21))
 (segment (start 114.7396 93.5227) (end 115.1926 94.6713) (width 0.6) (layer "F.Cu") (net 21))
 (segment (start 115.1926 94.6713) (end 115.5563 95.8513) (width 0.6) (layer "F.Cu") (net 21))
 (segment (start 115.5563 95.8513) (end 117.5391 95.3225) (width 0.6) (layer "F.Cu") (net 21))
 (segment (start 117.9572 97.5588) (end 115.9533 97.8312) (width 0.6) (layer "F.Cu") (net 20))
 (segment (start 115.9533 97.8312) (end 116.0767 99.135) (width 0.6) (layer "F.Cu") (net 20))
 (segment (start 116.0767 99.135) (end 116.0939 100.4445) (width 0.6) (layer "F.Cu") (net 20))
 (segment (start 116.0939 100.4445) (end 116.0045 101.7511) (width 0.6) (layer "F.Cu") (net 20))
 (segment (start 116.0045 101.7511) (end 118.0445 101.9743) (width 0.6) (layer "F.Cu") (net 20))
 (segment (start 117.6264 104.2106) (end 115.6594 103.7407) (width 0.6) (layer "F.Cu") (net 18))
 (segment (start 115.6594 103.7407) (end 115.3267 104.9298) (width 0.6) (layer "F.Cu") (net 18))
 (segment (start 115.3267 104.9298) (end 114.9038 106.0899) (width 0.6) (layer "F.Cu") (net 18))
 (segment (start 114.9038 106.0899) (end 114.3933 107.2141) (width 0.6) (layer "F.Cu") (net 18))
 (segment (start 114.3933 107.2141) (end 113.7981 108.296) (width 0.6) (layer "F.Cu") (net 18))
 (segment (start 113.7981 108.296) (end 113.1217 109.329) (width 0.6) (layer "F.Cu") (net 18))
 (segment (start 113.1217 109.329) (end 112.3682 110.3072) (width 0.6) (layer "F.Cu") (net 18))
 (segment (start 112.3682 110.3072) (end 111.5419 111.2247) (width 0.6) (layer "F.Cu") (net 18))
 (segment (start 111.5419 111.2247) (end 110.6478 112.0762) (width 0.6) (layer "F.Cu") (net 18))
 (segment (start 110.6478 112.0762) (end 112.005 113.6155) (width 0.6) (layer "F.Cu") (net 18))
 (segment (start 110.1895 114.9865) (end 109.0524 113.3141) (width 0.6) (layer "F.Cu") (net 16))
 (segment (start 109.0524 113.3141) (end 108.0054 113.9687) (width 0.6) (layer "F.Cu") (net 16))
 (segment (start 108.0054 113.9687) (end 106.9114 114.5411) (width 0.6) (layer "F.Cu") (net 16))
 (segment (start 106.9114 114.5411) (end 105.7766 115.028) (width 0.6) (layer "F.Cu") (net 16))
 (segment (start 105.7766 115.028) (end 104.6079 115.4265) (width 0.6) (layer "F.Cu") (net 16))
 (segment (start 104.6079 115.4265) (end 103.4122 115.7343) (width 0.6) (layer "F.Cu") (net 16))
 (segment (start 103.4122 115.7343) (end 102.1963 115.9495) (width 0.6) (layer "F.Cu") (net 16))
 (segment (start 102.1963 115.9495) (end 100.9675 116.0709) (width 0.6) (layer "F.Cu") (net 16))
 (segment (start 100.9675 116.0709) (end 99.733 116.0978) (width 0.6) (layer "F.Cu") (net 16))
 (segment (start 99.733 116.0978) (end 99.699 118.1497) (width 0.6) (layer "F.Cu") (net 16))
 (segment (start 97.4337 117.9398) (end 97.7201 115.9378) (width 0.6) (layer "F.Cu") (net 14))
 (segment (start 97.7201 115.9378) (end 96.5054 115.7162) (width 0.6) (layer "F.Cu") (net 14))
 (segment (start 96.5054 115.7162) (end 95.3112 115.4021) (width 0.6) (layer "F.Cu") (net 14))
 (segment (start 95.3112 115.4021) (end 94.1447 114.9975) (width 0.6) (layer "F.Cu") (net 14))
 (segment (start 94.1447 114.9975) (end 93.0125 114.5047) (width 0.6) (layer "F.Cu") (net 14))
 (segment (start 93.0125 114.5047) (end 91.9215 113.9265) (width 0.6) (layer "F.Cu") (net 14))
 (segment (start 91.9215 113.9265) (end 90.878 113.2664) (width 0.6) (layer "F.Cu") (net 14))
 (segment (start 90.878 113.2664) (end 89.8881 112.5283) (width 0.6) (layer "F.Cu") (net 14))
 (segment (start 89.8881 112.5283) (end 88.9577 111.7166) (width 0.6) (layer "F.Cu") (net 14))
 (segment (start 88.9577 111.7166) (end 87.5502 113.21) (width 0.6) (layer "F.Cu") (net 14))
 (segment (start 82.6256 94.7436) (end 82.0761 97.481) (width 0.6) (layer "F.Cu") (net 11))
 (segment (start 82.0761 97.481) (end 87.6924 98.4888) (width 0.6) (layer "F.Cu") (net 11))
 (segment (start 87.6924 98.4888) (end 89.6 98) (width 0.6) (layer "F.Cu") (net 11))
 (segment (start 89.6 98) (end 91.4 98) (width 0.6) (layer "F.Cu") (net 11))
 (segment (start 82.7972 105.6993) (end 82.0761 102.519) (width 0.6) (layer "F.Cu") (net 9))
 (segment (start 82.0761 102.519) (end 87.6924 101.5112) (width 0.6) (layer "F.Cu") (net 9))
 (segment (start 87.6924 101.5112) (end 89.6 102) (width 0.6) (layer "F.Cu") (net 9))
 (segment (start 89.6 102) (end 91.4 102) (width 0.6) (layer "F.Cu") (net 9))
 (segment (start 91.4 98) (end 94.4 98) (width 0.6) (layer "F.Cu") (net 11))
 (segment (start 85.6976 88.8222) (end 87.3146 90.0859) (width 0.6) (layer "F.Cu") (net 11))
 (segment (start 87.3146 90.0859) (end 94.4 98) (width 0.6) (layer "F.Cu") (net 11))
 (segment (start 86.0176 111.5288) (end 87.578 110.2422) (width 0.6) (layer "F.Cu") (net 10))
 (segment (start 87.578 110.2422) (end 94.4 102) (width 0.6) (layer "F.Cu") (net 10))
 (segment (start 101.7 100.8) (end 103 100.8) (width 0.3) (layer "F.Cu") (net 1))
 (segment (start 103 100.8) (end 103 101.6) (width 0.3) (layer "F.Cu") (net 1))
 (segment (start 103 101.6) (end 104.7 101.6) (width 0.3) (layer "F.Cu") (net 1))
 (segment (start 101.7 102.4) (end 103 102.4) (width 0.3) (layer "F.Cu") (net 2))
 (segment (start 103 102.4) (end 103 103.3) (width 0.3) (layer "F.Cu") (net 2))
 (segment (start 103 103.3) (end 106.3 103.3) (width 0.3) (layer "F.Cu") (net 2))
 (segment (start 106.3 103.3) (end 106.3 102.75) (width 0.3) (layer "F.Cu") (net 2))
 (segment (start 101.7 104) (end 107.9 104) (width 0.3) (layer "F.Cu") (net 3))
 (segment (start 107.9 104) (end 107.9 102.75) (width 0.3) (layer "F.Cu") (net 3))
 (segment (start 101.7 105.6) (end 108.5 105.6) (width 0.3) (layer "F.Cu") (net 4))
 (segment (start 108.5 105.6) (end 108.5 104.6) (width 0.3) (layer "F.Cu") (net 4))
 (segment (start 108.5 104.6) (end 109.5 104.6) (width 0.3) (layer "F.Cu") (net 4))
 (segment (start 109.5 104.6) (end 109.5 102.75) (width 0.3) (layer "F.Cu") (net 4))
 (segment (start 101.7 99.2) (end 103 99.2) (width 0.3) (layer "F.Cu") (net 5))
 (segment (start 103 99.2) (end 103 98.4) (width 0.3) (layer "F.Cu") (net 5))
 (segment (start 103 98.4) (end 104.7 98.4) (width 0.3) (layer "F.Cu") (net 5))
 (segment (start 101.7 97.6) (end 103 97.6) (width 0.3) (layer "F.Cu") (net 6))
 (segment (start 103 97.6) (end 103 96.7) (width 0.3) (layer "F.Cu") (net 6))
 (segment (start 103 96.7) (end 106.3 96.7) (width 0.3) (layer "F.Cu") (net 6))
 (segment (start 106.3 96.7) (end 106.3 97.25) (width 0.3) (layer "F.Cu") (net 6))
 (segment (start 101.7 96) (end 107.9 96) (width 0.3) (layer "F.Cu") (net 7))
 (segment (start 107.9 96) (end 107.9 97.25) (width 0.3) (layer "F.Cu") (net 7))
 (segment (start 101.7 94.4) (end 108.5 94.4) (width 0.3) (layer "F.Cu") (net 8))
 (segment (start 108.5 94.4) (end 108.5 95.4) (width 0.3) (layer "F.Cu") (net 8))
 (segment (start 108.5 95.4) (end 109.5 95.4) (width 0.3) (layer "F.Cu") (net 8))
 (segment (start 109.5 95.4) (end 109.5 97.25) (width 0.3) (layer "F.Cu") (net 8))
 (segment (start 101.7 105.6) (end 101.7 108.2) (width 0.3) (layer "F.Cu") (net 4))
 (segment (start 101.7 108.2) (end 98.3 108.2) (width 0.3) (layer "F.Cu") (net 4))
 (segment (start 98.3 108.2) (end 98.3 103.91) (width 0.3) (layer "F.Cu") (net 4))
 (segment (start 98.3 102.89) (end 98.3 100.8) (width 0.3) (layer "F.Cu") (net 12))
 (segment (start 98.3 100.8) (end 98.3 99.2) (width 0.3) (layer "F.Cu") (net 12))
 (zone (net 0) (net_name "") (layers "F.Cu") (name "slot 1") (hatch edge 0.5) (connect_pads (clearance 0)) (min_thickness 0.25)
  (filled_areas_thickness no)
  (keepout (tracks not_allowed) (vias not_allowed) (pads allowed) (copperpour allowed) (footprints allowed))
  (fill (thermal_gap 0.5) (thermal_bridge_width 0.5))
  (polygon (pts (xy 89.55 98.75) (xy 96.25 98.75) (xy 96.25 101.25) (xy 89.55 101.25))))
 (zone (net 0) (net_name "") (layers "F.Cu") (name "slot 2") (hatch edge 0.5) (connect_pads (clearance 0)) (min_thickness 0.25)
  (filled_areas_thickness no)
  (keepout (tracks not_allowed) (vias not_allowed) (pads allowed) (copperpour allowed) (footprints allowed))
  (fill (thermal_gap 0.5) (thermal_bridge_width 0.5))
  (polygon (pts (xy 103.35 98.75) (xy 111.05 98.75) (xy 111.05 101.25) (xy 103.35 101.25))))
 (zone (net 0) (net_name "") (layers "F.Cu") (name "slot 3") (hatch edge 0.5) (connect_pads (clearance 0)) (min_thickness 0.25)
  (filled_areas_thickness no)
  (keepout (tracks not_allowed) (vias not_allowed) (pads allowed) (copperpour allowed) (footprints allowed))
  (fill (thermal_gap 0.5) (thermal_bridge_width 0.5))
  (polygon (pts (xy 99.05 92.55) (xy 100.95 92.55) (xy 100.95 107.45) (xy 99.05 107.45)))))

